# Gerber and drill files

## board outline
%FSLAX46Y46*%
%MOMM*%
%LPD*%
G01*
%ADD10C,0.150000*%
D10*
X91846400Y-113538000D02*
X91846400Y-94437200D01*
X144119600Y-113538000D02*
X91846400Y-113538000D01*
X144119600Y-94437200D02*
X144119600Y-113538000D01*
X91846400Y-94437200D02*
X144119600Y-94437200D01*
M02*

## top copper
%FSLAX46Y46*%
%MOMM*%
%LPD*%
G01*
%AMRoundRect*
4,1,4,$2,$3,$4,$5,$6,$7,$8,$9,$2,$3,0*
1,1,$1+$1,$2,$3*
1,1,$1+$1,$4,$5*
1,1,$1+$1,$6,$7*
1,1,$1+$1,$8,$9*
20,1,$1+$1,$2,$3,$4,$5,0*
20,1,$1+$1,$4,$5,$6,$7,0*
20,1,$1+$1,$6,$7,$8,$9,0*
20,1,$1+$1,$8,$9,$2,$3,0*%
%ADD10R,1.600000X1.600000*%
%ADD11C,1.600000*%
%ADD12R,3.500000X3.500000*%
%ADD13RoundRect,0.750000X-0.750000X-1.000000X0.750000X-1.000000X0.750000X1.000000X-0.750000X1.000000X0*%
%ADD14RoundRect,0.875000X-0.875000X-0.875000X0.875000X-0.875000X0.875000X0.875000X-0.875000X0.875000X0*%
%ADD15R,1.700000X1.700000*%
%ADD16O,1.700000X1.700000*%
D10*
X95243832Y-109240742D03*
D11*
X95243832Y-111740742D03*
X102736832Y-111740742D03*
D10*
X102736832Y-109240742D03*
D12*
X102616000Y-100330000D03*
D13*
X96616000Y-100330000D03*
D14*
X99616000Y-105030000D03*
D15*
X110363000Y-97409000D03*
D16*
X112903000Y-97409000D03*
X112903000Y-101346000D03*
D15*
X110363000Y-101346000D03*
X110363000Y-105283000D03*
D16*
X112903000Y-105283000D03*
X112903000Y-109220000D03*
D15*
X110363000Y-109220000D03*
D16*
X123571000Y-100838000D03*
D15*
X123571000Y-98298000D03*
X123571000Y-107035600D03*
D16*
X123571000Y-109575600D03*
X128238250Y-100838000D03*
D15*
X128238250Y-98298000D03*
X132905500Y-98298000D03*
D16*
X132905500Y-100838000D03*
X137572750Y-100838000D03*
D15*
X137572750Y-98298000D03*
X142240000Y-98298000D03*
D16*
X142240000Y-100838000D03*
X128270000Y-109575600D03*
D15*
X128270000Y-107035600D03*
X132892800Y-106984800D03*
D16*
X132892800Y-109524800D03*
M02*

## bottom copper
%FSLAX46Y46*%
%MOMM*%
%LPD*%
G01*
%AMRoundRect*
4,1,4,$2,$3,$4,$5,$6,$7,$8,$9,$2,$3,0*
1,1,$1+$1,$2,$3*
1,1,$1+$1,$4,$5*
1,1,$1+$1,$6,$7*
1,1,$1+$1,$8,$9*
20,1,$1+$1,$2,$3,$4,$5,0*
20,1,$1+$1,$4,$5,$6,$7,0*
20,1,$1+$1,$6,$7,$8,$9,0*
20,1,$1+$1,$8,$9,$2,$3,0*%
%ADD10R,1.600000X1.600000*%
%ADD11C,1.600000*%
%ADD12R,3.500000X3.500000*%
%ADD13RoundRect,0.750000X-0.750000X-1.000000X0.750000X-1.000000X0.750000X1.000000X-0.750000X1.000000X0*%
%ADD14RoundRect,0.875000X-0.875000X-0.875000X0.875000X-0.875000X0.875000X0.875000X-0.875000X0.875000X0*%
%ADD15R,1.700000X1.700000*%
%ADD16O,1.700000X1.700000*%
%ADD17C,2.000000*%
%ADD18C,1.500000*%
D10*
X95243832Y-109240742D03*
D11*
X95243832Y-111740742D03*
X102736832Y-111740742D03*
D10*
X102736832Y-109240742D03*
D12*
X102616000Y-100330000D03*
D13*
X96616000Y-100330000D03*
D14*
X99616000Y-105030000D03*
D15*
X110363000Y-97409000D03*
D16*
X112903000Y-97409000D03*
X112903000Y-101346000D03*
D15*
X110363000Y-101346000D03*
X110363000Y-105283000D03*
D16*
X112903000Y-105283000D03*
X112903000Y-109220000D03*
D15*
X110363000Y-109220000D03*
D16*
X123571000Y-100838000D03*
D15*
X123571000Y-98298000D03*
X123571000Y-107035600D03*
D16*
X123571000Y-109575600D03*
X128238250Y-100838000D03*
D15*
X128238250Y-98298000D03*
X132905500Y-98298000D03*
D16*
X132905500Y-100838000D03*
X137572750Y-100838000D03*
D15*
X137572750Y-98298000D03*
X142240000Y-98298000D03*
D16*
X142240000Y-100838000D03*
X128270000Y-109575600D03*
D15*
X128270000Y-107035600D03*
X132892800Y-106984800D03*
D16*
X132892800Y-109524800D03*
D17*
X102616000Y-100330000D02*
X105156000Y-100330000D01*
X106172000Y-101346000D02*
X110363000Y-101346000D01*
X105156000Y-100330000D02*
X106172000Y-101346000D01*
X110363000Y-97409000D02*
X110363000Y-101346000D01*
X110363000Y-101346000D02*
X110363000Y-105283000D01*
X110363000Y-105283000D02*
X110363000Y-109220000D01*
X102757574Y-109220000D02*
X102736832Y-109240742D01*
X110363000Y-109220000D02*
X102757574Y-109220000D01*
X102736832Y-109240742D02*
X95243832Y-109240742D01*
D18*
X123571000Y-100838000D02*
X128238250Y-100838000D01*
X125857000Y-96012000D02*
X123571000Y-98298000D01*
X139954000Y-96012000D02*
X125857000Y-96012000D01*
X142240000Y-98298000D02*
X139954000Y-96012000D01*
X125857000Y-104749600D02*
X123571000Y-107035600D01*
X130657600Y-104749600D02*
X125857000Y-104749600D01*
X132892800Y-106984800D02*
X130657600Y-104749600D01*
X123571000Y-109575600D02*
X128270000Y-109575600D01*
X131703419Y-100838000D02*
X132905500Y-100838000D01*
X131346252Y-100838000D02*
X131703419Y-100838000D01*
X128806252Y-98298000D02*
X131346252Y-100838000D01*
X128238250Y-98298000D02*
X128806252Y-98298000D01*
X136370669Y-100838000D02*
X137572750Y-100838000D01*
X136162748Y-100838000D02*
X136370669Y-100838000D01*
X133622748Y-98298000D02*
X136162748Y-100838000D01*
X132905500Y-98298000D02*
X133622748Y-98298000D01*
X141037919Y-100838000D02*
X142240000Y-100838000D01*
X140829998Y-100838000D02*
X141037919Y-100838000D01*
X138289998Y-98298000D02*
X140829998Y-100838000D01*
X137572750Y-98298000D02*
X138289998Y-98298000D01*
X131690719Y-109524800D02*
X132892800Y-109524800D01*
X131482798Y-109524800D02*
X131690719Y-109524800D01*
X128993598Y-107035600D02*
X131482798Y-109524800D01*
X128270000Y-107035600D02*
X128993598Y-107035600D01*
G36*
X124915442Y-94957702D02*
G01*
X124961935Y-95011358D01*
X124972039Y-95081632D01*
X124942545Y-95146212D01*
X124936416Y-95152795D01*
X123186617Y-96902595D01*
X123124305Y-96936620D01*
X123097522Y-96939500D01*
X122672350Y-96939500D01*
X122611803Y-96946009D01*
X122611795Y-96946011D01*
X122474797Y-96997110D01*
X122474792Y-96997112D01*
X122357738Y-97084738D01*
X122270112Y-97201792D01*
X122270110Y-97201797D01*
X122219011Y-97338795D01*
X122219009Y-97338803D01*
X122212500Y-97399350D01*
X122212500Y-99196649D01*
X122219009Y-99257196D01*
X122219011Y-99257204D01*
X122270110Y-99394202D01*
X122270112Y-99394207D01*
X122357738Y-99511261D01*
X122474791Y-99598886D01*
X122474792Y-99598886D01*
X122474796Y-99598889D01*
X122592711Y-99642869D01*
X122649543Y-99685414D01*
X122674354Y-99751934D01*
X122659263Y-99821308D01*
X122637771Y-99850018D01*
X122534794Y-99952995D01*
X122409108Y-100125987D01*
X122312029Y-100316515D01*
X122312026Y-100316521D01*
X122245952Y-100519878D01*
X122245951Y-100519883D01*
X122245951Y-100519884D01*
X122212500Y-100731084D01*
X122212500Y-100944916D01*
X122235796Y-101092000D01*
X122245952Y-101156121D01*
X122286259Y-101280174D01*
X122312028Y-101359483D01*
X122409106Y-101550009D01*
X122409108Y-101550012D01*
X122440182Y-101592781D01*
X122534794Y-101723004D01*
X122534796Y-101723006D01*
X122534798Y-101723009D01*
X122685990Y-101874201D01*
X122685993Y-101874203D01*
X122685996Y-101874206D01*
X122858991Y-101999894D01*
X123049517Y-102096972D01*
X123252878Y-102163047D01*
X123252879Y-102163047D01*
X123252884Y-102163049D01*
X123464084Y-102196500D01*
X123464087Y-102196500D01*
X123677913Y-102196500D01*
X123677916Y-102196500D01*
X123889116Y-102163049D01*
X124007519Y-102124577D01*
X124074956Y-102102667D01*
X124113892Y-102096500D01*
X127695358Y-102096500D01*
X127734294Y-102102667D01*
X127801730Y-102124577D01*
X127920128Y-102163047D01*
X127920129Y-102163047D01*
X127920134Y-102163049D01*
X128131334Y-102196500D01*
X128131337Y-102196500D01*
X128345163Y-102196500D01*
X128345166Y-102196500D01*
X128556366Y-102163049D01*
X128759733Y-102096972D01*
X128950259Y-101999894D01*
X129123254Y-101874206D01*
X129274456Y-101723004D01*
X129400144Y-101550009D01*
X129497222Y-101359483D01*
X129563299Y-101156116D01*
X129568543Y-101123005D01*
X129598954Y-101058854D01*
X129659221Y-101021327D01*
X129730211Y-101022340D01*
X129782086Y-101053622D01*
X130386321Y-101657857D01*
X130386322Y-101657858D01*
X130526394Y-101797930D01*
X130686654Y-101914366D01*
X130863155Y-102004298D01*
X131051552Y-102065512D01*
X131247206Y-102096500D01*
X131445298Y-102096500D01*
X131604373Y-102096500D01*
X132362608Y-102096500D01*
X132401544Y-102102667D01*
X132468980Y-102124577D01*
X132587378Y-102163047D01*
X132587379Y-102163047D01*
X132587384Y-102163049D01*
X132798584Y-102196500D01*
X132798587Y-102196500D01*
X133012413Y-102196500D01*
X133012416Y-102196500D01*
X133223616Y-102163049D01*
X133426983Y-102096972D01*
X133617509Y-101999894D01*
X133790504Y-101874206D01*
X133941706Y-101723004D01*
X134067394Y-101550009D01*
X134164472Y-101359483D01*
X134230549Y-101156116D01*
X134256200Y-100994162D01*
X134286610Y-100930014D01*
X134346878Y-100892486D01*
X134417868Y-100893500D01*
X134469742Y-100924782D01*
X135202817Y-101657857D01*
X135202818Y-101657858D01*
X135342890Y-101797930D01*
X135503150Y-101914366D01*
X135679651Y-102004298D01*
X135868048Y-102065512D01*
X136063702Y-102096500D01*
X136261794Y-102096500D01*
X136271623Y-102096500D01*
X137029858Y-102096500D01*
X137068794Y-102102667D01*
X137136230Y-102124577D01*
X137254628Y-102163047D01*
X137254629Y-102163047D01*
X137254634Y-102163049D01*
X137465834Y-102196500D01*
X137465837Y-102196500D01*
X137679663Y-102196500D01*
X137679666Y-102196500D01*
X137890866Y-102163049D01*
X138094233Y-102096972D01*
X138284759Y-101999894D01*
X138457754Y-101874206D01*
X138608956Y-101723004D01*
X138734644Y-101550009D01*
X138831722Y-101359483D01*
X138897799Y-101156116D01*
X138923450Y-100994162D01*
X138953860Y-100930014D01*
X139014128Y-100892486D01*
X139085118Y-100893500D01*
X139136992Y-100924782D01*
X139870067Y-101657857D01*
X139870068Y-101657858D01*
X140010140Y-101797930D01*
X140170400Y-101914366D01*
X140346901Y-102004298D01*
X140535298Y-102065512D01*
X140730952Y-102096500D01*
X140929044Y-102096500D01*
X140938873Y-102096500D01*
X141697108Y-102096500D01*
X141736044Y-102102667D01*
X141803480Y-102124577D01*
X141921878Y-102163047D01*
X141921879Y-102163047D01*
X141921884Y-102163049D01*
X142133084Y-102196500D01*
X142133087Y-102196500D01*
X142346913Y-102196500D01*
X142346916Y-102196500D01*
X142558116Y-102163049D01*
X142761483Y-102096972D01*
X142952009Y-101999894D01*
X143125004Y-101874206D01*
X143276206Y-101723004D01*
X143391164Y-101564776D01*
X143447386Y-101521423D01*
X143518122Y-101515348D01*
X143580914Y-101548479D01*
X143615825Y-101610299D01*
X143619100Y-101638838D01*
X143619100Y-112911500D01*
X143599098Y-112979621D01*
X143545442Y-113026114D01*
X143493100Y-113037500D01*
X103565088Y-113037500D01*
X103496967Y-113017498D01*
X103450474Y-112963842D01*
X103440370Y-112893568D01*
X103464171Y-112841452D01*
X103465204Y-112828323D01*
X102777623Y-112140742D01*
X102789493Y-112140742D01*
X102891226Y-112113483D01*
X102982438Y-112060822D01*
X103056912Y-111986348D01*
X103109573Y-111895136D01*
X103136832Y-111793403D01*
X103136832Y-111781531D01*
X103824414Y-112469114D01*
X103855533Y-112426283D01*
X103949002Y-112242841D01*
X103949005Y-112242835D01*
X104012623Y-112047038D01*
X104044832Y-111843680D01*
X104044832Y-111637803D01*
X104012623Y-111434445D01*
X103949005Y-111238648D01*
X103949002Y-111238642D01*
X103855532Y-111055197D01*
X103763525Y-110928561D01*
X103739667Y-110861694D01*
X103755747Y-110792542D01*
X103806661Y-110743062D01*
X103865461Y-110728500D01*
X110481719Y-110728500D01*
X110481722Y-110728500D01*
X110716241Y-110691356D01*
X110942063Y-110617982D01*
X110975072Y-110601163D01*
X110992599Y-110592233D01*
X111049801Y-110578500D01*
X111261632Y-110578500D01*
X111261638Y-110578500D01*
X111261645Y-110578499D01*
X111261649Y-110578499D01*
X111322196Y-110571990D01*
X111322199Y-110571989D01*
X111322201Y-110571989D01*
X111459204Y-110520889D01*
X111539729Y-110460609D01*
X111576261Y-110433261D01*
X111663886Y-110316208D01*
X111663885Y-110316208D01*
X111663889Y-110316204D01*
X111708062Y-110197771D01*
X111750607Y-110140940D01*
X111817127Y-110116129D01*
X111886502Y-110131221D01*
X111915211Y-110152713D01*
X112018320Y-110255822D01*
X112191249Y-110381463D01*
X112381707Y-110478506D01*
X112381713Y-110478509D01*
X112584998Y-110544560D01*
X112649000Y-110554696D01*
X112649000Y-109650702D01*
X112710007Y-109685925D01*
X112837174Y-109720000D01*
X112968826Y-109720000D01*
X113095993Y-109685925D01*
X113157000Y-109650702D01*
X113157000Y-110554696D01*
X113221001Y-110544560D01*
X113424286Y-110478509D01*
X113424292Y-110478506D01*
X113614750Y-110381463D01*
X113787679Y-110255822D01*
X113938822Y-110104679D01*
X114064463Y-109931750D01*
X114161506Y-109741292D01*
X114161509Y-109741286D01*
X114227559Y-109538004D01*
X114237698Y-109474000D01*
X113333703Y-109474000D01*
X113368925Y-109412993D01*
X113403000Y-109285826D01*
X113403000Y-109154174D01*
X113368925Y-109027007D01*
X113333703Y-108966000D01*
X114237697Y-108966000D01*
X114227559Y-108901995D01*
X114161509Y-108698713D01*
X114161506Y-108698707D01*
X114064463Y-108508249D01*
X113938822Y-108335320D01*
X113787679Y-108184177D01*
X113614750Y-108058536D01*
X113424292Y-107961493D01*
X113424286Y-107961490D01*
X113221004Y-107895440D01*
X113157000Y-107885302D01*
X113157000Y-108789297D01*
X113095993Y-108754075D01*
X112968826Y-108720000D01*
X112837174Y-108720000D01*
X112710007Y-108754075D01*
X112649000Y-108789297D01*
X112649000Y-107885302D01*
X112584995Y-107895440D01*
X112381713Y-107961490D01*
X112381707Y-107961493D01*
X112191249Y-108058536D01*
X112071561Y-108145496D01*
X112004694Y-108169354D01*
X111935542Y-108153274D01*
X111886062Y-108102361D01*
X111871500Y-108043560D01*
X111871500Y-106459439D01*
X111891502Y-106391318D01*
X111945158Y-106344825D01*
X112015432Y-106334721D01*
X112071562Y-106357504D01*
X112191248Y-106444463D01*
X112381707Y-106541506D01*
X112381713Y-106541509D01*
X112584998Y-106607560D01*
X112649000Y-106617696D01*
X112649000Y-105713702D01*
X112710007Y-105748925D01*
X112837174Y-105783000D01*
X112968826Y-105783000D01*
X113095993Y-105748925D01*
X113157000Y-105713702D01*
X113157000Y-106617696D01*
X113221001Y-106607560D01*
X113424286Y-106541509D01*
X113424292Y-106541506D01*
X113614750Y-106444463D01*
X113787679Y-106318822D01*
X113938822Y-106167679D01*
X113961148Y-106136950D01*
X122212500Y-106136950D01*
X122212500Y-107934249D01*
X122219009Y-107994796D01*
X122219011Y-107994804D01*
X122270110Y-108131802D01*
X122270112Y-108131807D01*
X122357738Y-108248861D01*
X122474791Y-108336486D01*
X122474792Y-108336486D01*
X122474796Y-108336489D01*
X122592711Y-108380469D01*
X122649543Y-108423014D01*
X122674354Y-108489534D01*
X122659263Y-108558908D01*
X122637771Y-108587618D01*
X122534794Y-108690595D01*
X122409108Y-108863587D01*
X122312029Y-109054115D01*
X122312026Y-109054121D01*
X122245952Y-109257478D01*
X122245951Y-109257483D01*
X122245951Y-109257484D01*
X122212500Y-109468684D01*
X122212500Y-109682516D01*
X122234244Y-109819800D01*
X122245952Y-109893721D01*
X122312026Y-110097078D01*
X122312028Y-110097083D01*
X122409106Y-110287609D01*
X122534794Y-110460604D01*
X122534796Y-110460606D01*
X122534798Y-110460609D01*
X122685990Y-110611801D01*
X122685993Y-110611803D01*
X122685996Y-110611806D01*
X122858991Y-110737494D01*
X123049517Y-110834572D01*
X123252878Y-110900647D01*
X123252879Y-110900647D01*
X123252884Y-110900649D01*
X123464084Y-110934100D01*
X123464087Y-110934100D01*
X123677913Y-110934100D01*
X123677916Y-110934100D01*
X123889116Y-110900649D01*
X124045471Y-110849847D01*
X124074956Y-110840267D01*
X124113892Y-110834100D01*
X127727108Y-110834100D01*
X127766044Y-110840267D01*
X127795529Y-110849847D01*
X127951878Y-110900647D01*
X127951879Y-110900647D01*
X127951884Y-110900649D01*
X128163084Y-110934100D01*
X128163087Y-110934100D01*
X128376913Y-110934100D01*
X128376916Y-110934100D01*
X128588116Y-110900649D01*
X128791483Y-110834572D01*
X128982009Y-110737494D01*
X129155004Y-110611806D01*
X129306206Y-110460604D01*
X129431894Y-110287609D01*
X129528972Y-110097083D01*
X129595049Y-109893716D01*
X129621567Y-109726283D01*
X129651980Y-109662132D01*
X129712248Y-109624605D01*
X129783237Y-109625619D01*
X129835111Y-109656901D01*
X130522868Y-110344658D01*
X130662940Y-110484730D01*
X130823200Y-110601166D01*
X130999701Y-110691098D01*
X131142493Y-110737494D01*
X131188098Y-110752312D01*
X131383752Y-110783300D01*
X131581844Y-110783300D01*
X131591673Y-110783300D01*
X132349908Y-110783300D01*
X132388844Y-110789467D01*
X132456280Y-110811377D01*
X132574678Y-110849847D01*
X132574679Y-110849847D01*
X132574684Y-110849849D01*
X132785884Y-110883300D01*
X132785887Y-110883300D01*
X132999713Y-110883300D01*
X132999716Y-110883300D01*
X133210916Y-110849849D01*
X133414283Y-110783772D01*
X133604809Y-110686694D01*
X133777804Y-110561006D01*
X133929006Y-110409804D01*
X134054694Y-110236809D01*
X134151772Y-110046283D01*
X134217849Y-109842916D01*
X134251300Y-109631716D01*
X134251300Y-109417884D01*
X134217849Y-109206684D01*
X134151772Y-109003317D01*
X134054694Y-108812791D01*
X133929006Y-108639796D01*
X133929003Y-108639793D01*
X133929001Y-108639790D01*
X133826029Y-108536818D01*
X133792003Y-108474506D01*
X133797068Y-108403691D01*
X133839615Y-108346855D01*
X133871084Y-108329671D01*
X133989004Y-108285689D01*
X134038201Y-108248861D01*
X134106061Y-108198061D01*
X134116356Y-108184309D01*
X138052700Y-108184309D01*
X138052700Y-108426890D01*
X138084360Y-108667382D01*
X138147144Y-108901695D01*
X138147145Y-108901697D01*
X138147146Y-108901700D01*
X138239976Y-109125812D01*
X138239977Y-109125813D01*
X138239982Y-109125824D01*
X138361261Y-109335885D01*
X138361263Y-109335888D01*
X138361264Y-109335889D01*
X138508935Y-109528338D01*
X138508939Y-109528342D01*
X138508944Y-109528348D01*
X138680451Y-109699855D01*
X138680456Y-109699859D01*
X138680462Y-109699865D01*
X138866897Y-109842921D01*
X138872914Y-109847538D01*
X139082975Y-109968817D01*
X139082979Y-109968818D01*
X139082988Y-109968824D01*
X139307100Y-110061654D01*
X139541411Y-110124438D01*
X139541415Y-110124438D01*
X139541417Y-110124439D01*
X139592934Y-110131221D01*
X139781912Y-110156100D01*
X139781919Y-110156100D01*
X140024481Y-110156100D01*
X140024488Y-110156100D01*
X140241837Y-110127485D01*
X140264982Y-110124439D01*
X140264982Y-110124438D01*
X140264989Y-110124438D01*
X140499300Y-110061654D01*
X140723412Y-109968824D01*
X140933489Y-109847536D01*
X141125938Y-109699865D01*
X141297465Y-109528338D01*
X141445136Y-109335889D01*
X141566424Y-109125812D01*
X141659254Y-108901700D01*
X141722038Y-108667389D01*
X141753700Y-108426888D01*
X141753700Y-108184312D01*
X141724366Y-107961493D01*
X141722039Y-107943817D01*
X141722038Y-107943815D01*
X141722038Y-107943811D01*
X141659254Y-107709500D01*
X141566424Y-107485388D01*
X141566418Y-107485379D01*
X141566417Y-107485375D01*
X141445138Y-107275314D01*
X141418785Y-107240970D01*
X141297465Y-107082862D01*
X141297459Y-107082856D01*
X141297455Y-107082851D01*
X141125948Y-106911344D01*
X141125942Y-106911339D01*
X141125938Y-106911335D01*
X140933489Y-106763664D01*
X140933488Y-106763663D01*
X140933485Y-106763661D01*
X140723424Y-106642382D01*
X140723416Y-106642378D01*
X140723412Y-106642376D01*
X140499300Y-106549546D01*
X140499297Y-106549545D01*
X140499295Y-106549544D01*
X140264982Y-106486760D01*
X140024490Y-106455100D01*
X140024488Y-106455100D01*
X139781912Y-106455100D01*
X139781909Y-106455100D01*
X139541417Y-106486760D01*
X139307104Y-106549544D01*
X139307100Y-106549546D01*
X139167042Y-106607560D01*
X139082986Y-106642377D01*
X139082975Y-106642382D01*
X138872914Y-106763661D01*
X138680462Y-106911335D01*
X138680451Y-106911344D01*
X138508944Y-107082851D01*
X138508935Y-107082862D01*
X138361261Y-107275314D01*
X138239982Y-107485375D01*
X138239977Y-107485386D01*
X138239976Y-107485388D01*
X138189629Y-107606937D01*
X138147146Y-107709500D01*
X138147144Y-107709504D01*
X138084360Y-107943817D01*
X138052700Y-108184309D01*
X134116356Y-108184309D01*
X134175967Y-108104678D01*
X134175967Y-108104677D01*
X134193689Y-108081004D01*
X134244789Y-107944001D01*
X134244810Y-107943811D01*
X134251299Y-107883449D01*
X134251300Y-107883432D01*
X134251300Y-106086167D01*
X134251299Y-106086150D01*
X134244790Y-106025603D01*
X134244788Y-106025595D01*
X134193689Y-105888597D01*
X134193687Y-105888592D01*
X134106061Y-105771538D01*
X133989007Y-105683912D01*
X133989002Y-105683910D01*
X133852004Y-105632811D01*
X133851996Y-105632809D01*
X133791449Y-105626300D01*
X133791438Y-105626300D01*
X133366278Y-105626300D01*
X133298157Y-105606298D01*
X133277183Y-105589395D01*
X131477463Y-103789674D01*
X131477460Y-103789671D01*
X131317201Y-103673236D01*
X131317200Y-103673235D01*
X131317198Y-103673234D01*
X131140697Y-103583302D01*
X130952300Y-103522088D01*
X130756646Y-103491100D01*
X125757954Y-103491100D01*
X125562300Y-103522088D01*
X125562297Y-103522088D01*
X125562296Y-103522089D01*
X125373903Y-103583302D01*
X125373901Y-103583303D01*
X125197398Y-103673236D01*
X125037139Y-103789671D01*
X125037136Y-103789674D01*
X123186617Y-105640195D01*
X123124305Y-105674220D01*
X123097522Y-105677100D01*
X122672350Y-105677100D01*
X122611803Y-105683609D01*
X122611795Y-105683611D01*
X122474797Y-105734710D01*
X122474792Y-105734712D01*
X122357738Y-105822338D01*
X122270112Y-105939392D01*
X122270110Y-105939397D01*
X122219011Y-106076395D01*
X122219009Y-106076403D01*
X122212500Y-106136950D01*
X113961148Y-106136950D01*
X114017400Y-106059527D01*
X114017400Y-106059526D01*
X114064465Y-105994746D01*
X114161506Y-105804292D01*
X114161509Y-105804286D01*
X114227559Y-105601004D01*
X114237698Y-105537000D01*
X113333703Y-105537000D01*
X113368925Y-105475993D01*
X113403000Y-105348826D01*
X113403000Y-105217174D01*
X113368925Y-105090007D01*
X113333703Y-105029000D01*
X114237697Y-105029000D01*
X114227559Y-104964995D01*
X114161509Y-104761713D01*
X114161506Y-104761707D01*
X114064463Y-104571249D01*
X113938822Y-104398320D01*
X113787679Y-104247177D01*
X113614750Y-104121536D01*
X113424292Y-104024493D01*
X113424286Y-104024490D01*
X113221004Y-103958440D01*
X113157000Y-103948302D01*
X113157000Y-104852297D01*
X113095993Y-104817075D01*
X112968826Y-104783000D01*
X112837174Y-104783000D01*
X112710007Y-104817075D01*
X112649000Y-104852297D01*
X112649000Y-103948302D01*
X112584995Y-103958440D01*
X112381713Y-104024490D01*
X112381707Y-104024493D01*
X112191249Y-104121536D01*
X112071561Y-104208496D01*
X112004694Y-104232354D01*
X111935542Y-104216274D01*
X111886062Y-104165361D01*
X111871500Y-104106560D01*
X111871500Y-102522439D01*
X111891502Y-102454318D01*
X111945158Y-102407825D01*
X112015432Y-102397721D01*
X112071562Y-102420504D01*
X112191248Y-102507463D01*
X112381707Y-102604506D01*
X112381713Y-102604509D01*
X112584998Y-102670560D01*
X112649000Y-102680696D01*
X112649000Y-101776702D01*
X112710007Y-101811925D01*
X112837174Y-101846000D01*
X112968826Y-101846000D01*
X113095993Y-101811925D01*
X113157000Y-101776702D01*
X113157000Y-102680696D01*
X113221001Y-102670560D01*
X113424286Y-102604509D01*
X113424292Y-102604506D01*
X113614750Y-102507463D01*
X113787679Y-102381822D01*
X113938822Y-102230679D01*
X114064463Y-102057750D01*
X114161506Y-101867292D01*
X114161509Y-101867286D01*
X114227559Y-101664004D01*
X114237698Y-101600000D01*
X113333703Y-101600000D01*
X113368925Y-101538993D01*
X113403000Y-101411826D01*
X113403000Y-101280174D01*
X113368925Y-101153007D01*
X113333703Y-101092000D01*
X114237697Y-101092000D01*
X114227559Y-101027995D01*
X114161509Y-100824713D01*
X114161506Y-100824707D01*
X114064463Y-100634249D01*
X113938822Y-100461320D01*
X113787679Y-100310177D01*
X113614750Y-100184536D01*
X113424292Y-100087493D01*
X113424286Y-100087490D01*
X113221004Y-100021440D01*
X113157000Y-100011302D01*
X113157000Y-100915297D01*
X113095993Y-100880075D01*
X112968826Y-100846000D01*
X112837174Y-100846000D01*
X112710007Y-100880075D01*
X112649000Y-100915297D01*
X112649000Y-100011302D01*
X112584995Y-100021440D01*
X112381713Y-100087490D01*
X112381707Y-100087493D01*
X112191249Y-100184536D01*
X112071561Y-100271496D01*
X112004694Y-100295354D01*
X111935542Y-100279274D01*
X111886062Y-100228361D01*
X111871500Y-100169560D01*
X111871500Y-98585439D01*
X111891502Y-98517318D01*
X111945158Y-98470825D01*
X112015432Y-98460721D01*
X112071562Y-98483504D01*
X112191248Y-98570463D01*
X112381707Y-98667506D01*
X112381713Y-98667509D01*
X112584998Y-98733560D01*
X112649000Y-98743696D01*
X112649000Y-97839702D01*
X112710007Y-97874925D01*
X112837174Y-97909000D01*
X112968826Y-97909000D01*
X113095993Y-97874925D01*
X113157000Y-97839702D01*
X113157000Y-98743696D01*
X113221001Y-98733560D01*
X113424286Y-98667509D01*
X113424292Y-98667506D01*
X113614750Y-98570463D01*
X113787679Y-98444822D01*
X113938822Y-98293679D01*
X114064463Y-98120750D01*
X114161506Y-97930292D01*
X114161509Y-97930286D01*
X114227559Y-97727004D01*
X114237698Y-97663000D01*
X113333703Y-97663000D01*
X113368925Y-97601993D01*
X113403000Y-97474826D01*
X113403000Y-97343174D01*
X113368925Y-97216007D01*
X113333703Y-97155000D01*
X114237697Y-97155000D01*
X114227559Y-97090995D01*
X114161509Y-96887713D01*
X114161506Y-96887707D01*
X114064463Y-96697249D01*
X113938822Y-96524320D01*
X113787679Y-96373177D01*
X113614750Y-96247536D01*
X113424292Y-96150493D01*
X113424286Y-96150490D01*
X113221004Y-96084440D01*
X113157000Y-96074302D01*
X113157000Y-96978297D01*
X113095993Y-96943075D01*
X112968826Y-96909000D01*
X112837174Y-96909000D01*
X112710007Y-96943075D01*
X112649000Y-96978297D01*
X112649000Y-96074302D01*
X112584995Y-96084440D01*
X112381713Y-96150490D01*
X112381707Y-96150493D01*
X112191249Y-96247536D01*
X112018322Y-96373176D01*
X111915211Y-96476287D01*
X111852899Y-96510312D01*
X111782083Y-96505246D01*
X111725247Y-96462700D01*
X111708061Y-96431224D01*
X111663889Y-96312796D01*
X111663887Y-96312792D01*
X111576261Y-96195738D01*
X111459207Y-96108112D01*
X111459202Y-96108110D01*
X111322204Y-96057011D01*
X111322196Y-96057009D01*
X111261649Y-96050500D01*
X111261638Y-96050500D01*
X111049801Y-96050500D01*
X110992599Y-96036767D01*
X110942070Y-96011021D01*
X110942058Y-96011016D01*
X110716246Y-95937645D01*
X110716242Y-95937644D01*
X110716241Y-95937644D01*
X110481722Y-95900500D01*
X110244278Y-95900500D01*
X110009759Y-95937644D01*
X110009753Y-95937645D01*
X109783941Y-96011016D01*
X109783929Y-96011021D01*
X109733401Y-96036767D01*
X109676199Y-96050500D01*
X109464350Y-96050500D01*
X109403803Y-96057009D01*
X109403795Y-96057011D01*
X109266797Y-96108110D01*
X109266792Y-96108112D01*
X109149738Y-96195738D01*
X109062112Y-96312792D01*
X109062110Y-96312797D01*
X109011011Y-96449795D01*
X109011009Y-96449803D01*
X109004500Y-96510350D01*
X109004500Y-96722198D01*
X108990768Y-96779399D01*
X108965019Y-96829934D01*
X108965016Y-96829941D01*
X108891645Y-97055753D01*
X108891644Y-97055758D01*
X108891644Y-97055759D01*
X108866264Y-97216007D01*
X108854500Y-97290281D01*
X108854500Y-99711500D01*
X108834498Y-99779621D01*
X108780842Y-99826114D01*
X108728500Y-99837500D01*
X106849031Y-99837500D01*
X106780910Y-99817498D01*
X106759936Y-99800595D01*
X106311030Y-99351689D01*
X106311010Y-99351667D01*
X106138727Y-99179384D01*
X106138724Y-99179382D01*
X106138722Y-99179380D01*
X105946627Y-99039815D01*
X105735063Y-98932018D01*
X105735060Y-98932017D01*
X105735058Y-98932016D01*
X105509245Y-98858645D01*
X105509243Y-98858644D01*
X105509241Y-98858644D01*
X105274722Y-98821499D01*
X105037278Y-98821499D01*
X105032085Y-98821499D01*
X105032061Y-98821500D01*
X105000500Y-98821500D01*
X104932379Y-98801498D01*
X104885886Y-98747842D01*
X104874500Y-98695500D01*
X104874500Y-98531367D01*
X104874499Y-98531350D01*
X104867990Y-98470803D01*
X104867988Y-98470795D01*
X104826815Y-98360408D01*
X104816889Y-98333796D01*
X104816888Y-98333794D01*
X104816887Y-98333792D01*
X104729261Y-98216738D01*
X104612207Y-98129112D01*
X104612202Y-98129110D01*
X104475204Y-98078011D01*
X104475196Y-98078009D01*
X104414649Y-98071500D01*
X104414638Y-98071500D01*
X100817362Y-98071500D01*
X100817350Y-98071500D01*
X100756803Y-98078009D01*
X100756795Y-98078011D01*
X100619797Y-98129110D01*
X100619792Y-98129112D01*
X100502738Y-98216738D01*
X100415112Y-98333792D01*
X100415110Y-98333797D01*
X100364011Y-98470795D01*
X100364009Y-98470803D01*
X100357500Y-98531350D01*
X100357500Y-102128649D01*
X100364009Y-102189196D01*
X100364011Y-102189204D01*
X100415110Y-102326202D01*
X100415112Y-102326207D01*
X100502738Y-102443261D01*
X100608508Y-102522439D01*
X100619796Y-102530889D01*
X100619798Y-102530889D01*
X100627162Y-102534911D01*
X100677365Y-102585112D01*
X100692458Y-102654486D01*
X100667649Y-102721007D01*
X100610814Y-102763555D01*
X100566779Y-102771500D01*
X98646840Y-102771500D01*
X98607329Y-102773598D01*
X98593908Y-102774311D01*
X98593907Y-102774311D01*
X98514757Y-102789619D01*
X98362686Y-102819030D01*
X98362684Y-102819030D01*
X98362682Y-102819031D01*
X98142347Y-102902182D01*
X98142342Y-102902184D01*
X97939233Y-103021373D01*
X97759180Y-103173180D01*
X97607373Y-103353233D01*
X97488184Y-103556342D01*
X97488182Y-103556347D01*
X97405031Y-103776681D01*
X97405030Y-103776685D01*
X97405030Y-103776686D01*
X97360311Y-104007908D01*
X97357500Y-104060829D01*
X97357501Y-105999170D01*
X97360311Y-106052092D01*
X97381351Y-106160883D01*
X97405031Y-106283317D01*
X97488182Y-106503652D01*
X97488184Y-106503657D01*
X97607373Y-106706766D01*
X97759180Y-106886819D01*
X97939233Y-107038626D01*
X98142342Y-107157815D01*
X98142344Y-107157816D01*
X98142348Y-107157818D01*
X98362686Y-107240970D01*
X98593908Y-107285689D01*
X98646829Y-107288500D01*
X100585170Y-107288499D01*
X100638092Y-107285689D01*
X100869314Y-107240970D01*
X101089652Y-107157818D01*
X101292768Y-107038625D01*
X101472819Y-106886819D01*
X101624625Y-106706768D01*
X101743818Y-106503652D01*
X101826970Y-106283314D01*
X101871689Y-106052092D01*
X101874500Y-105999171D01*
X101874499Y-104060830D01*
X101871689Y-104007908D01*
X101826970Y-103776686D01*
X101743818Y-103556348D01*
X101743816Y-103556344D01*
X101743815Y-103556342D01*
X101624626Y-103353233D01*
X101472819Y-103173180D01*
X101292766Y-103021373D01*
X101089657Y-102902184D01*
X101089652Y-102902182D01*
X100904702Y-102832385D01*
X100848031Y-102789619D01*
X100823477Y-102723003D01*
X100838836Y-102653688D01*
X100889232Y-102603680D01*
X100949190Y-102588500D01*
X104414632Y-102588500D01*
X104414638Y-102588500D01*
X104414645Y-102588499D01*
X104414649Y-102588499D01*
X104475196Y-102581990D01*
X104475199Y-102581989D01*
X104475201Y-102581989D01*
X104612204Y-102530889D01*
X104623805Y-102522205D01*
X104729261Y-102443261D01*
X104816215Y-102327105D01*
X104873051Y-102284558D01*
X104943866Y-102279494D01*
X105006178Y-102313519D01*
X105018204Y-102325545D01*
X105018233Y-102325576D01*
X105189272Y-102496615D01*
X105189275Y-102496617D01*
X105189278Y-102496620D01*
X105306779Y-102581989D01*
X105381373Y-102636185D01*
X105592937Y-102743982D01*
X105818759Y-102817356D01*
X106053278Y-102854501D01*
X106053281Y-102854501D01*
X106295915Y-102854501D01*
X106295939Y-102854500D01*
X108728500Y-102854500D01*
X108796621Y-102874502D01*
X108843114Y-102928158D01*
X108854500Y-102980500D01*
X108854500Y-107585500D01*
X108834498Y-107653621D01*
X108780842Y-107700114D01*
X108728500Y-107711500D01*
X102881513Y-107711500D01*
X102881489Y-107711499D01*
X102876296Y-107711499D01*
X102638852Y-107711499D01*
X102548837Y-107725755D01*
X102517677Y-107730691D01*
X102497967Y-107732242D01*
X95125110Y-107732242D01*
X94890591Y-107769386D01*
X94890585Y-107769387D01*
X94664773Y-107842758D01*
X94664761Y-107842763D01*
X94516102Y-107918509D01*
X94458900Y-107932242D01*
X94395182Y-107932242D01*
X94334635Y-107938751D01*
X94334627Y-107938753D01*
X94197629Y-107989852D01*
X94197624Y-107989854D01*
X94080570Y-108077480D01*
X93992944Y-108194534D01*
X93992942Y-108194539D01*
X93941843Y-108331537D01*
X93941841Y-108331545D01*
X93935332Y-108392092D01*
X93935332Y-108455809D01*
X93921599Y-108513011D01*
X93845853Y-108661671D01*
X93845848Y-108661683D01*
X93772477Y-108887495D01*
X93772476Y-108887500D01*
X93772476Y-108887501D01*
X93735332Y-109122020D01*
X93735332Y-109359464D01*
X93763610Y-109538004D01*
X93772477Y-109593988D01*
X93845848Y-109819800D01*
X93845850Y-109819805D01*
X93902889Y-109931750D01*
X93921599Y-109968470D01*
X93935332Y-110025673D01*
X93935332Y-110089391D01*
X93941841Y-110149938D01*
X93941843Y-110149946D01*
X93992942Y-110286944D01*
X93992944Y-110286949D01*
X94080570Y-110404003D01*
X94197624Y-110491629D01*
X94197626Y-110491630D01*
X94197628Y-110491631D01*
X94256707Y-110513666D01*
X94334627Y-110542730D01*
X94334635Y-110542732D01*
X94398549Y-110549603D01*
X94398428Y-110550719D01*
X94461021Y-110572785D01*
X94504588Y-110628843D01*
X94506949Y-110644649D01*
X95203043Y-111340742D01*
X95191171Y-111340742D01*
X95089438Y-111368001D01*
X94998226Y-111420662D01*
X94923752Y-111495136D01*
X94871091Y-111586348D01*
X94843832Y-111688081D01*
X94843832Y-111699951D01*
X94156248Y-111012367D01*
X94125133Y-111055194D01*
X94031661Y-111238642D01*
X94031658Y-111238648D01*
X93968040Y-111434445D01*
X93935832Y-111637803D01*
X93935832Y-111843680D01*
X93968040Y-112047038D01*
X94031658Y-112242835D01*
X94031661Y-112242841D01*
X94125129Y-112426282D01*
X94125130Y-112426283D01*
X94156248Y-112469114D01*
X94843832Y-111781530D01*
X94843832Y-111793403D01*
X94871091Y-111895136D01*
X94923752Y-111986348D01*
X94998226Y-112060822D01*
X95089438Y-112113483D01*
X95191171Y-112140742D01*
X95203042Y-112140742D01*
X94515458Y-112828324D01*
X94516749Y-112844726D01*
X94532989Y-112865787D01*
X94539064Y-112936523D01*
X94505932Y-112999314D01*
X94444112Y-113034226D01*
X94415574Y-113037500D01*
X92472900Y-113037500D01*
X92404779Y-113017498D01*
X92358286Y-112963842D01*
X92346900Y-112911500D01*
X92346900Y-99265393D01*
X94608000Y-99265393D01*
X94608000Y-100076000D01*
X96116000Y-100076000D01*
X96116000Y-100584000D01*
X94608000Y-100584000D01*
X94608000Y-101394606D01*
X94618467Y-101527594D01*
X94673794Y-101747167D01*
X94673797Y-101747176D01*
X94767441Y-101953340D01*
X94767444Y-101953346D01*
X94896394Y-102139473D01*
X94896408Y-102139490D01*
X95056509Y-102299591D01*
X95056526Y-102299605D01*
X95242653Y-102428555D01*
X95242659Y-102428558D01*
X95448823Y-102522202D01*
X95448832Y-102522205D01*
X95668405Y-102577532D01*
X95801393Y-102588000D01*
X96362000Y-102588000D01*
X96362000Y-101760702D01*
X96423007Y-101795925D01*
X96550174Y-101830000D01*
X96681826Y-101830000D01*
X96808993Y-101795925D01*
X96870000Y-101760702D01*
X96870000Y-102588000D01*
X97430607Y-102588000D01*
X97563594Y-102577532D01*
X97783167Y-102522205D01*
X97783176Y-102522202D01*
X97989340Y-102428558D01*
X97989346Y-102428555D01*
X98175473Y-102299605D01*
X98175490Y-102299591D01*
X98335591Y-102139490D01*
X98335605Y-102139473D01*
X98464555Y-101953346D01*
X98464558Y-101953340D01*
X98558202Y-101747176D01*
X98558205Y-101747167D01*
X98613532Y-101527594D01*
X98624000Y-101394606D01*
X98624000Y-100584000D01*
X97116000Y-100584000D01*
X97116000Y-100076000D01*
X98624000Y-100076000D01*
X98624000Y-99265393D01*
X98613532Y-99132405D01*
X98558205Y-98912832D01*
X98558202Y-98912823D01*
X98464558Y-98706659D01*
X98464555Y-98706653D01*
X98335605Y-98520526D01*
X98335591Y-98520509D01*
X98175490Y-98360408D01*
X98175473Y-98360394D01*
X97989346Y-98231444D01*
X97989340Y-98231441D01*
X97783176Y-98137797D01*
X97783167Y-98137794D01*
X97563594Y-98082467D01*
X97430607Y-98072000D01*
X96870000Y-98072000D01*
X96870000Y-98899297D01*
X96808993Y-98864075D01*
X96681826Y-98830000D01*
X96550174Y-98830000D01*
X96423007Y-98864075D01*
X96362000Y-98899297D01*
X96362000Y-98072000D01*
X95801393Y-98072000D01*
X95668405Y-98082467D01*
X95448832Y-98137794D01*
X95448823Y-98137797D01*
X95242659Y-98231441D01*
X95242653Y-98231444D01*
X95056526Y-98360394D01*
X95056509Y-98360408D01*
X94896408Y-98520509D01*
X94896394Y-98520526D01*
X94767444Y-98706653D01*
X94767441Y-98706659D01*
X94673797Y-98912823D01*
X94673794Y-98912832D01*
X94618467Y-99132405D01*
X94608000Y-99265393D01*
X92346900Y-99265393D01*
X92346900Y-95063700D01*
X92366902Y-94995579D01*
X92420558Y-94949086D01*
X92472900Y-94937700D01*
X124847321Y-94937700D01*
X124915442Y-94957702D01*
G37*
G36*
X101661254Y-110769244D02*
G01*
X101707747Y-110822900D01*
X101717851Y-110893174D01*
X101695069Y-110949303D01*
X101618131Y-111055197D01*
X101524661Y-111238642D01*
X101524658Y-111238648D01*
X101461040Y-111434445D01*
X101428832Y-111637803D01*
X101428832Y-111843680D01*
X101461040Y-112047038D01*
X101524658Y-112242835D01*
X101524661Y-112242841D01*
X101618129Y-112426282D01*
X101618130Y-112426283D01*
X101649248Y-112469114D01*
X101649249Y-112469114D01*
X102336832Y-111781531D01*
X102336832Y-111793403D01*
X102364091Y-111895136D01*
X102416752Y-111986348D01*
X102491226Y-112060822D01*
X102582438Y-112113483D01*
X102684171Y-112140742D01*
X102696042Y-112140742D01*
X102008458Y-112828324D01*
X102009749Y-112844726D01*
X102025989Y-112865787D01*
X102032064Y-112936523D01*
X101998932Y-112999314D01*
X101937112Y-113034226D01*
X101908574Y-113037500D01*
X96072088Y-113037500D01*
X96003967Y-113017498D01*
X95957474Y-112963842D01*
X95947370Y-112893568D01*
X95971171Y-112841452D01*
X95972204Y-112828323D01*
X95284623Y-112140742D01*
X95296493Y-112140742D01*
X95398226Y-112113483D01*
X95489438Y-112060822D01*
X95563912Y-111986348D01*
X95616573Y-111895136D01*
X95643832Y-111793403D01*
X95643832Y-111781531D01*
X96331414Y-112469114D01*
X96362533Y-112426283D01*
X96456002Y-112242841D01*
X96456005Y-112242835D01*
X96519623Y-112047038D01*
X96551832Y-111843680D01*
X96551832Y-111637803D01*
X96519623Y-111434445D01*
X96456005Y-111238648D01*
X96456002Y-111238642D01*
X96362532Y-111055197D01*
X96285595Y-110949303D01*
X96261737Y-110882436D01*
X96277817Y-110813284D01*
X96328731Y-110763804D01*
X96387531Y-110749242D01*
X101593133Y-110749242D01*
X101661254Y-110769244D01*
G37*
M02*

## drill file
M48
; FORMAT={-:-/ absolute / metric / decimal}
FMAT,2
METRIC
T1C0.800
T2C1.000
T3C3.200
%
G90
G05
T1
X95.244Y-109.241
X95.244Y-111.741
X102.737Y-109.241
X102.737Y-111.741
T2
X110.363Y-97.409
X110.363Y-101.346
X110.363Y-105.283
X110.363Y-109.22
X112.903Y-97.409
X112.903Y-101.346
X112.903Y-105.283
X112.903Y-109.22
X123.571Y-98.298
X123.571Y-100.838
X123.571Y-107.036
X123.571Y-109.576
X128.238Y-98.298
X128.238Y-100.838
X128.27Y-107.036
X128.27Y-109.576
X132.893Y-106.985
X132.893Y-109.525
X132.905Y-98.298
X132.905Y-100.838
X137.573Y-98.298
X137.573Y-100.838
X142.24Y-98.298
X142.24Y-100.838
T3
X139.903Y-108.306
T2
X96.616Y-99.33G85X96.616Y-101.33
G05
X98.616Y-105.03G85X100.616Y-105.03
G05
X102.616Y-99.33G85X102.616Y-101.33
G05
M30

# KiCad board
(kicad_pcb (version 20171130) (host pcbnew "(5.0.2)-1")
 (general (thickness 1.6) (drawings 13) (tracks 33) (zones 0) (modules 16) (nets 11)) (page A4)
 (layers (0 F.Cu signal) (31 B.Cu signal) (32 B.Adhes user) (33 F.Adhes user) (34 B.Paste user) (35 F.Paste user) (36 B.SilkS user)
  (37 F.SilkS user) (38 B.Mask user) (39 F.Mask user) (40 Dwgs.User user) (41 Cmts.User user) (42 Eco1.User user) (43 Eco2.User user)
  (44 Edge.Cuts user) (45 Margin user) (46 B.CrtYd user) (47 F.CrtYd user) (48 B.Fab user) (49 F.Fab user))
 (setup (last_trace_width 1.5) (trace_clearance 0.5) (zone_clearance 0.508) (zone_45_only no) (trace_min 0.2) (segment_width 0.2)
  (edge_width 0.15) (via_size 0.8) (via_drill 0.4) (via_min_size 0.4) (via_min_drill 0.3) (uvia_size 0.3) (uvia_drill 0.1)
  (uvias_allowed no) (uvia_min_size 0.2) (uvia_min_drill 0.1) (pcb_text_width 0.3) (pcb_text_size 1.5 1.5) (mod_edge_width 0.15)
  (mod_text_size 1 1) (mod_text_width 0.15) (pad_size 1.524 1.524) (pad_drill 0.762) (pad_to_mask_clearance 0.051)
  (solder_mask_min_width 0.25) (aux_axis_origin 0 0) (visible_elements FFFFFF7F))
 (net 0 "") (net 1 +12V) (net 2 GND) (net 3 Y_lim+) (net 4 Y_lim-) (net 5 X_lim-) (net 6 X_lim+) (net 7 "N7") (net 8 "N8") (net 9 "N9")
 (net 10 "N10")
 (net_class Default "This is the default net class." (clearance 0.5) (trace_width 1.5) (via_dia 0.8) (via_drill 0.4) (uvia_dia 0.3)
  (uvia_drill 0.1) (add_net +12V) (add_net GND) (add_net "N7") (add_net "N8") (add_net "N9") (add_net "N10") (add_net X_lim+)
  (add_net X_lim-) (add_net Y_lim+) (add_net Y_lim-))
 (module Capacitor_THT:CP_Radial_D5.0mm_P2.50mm (layer F.Cu) (at 95.243832 109.240742 270)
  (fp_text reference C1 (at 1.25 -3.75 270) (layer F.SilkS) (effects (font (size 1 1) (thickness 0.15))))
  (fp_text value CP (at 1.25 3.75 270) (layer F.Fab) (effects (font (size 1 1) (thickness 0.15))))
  (pad 1 thru_hole rect (at 0 0 270) (size 1.6 1.6) (drill 0.8) (layers *.Cu *.Mask) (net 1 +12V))
  (pad 2 thru_hole circle (at 2.5 0 270) (size 1.6 1.6) (drill 0.8) (layers *.Cu *.Mask) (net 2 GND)))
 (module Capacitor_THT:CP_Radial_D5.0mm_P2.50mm (layer F.Cu) (at 102.736832 109.240742 270)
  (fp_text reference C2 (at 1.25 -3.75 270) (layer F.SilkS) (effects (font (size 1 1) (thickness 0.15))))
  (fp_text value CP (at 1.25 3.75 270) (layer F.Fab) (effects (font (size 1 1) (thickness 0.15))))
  (pad 2 thru_hole circle (at 2.5 0 270) (size 1.6 1.6) (drill 0.8) (layers *.Cu *.Mask) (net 2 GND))
  (pad 1 thru_hole rect (at 0 0 270) (size 1.6 1.6) (drill 0.8) (layers *.Cu *.Mask) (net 1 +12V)))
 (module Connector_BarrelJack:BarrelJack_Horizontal (layer F.Cu) (at 102.616 100.33)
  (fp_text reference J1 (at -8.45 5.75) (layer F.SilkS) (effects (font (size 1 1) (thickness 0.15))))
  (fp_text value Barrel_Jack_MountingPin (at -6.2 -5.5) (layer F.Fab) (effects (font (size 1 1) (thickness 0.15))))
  (pad 1 thru_hole rect (at 0 0) (size 3.5 3.5) (drill oval 1 3) (layers *.Cu *.Mask) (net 1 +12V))
  (pad 2 thru_hole roundrect (at -6 0) (size 3 3.5) (drill oval 1 3) (layers *.Cu *.Mask) (roundrect_rratio 0.25) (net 2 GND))
  (pad 3 thru_hole roundrect (at -3 4.7) (size 3.5 3.5) (drill oval 3 1) (layers *.Cu *.Mask) (roundrect_rratio 0.25)))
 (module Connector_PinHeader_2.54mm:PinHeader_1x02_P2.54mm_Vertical (layer F.Cu) (at 110.363 97.409 90)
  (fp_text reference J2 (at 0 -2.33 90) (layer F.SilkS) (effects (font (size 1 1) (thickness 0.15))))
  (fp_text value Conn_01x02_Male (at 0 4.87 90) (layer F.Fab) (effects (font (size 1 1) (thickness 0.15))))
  (pad 1 thru_hole rect (at 0 0 90) (size 1.7 1.7) (drill 1) (layers *.Cu *.Mask) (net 1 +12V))
  (pad 2 thru_hole oval (at 0 2.54 90) (size 1.7 1.7) (drill 1) (layers *.Cu *.Mask) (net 2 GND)))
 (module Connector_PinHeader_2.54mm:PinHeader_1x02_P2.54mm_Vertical (layer F.Cu) (at 110.363 101.346 90)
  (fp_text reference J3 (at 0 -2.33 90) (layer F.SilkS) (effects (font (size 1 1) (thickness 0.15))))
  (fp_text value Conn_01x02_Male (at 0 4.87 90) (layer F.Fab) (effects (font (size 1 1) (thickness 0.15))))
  (pad 2 thru_hole oval (at 0 2.54 90) (size 1.7 1.7) (drill 1) (layers *.Cu *.Mask) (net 2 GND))
  (pad 1 thru_hole rect (at 0 0 90) (size 1.7 1.7) (drill 1) (layers *.Cu *.Mask) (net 1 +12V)))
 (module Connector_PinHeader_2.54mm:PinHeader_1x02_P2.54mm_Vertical (layer F.Cu) (at 110.363 105.283 90)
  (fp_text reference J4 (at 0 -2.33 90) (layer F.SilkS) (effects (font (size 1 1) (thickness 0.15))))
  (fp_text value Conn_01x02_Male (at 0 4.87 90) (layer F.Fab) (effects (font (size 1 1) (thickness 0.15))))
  (pad 1 thru_hole rect (at 0 0 90) (size 1.7 1.7) (drill 1) (layers *.Cu *.Mask) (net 1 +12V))
  (pad 2 thru_hole oval (at 0 2.54 90) (size 1.7 1.7) (drill 1) (layers *.Cu *.Mask) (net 2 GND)))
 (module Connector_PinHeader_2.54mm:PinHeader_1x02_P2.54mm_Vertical (layer F.Cu) (at 110.363 109.22 90)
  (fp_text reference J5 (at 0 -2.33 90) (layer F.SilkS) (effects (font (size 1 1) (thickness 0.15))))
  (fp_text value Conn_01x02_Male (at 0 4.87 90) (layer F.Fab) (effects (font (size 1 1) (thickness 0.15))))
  (pad 2 thru_hole oval (at 0 2.54 90) (size 1.7 1.7) (drill 1) (layers *.Cu *.Mask) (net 2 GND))
  (pad 1 thru_hole rect (at 0 0 90) (size 1.7 1.7) (drill 1) (layers *.Cu *.Mask) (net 1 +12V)))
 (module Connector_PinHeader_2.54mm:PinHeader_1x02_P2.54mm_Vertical (layer F.Cu) (at 123.571 98.298)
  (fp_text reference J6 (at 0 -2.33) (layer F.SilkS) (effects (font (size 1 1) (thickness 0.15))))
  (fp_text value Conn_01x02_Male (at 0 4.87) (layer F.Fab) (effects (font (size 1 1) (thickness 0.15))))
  (pad 2 thru_hole oval (at 0 2.54) (size 1.7 1.7) (drill 1) (layers *.Cu *.Mask) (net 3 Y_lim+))
  (pad 1 thru_hole rect (at 0 0) (size 1.7 1.7) (drill 1) (layers *.Cu *.Mask) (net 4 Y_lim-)))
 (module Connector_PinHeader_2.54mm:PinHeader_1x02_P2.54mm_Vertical (layer F.Cu) (at 123.571 107.0356)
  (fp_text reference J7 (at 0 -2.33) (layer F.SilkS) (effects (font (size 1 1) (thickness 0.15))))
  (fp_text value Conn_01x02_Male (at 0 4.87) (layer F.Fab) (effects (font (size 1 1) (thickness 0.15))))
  (pad 1 thru_hole rect (at 0 0) (size 1.7 1.7) (drill 1) (layers *.Cu *.Mask) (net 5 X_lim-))
  (pad 2 thru_hole oval (at 0 2.54) (size 1.7 1.7) (drill 1) (layers *.Cu *.Mask) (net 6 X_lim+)))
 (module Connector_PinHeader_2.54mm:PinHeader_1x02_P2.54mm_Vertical (layer F.Cu) (at 128.23825 98.298)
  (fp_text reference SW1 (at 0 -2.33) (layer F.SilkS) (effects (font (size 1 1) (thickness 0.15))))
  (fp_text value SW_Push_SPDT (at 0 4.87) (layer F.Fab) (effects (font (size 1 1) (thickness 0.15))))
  (pad 2 thru_hole oval (at 0 2.54) (size 1.7 1.7) (drill 1) (layers *.Cu *.Mask) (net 3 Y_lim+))
  (pad 1 thru_hole rect (at 0 0) (size 1.7 1.7) (drill 1) (layers *.Cu *.Mask) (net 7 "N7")))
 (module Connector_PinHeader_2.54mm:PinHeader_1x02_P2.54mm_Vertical (layer F.Cu) (at 132.9055 98.298)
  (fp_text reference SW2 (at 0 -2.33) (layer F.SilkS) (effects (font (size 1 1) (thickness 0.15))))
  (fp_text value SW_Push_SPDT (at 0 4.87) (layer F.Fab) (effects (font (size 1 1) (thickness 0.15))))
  (pad 1 thru_hole rect (at 0 0) (size 1.7 1.7) (drill 1) (layers *.Cu *.Mask) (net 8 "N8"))
  (pad 2 thru_hole oval (at 0 2.54) (size 1.7 1.7) (drill 1) (layers *.Cu *.Mask) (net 7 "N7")))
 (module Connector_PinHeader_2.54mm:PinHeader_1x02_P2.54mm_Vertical (layer F.Cu) (at 137.57275 98.298)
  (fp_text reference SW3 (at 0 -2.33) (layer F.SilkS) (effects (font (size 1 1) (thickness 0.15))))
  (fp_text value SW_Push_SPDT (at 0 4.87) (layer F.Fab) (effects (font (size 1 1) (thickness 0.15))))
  (pad 2 thru_hole oval (at 0 2.54) (size 1.7 1.7) (drill 1) (layers *.Cu *.Mask) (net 8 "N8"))
  (pad 1 thru_hole rect (at 0 0) (size 1.7 1.7) (drill 1) (layers *.Cu *.Mask) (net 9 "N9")))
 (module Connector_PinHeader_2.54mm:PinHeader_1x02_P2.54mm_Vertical (layer F.Cu) (at 142.24 98.298)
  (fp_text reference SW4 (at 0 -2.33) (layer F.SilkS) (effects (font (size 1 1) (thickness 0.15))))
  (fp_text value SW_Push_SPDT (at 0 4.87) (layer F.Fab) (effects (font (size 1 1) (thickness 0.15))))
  (pad 1 thru_hole rect (at 0 0) (size 1.7 1.7) (drill 1) (layers *.Cu *.Mask) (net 4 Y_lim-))
  (pad 2 thru_hole oval (at 0 2.54) (size 1.7 1.7) (drill 1) (layers *.Cu *.Mask) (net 9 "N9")))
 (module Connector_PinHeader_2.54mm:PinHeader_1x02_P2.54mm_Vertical (layer F.Cu) (at 128.27 107.0356)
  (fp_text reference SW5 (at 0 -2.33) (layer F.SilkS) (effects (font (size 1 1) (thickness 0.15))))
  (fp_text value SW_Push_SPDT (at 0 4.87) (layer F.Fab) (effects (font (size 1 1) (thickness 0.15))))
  (pad 2 thru_hole oval (at 0 2.54) (size 1.7 1.7) (drill 1) (layers *.Cu *.Mask) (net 6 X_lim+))
  (pad 1 thru_hole rect (at 0 0) (size 1.7 1.7) (drill 1) (layers *.Cu *.Mask) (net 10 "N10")))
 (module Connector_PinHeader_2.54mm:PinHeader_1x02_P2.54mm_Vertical (layer F.Cu) (at 132.8928 106.9848)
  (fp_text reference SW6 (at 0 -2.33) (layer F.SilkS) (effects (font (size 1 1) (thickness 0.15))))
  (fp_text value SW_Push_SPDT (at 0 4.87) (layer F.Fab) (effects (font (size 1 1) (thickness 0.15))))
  (pad 1 thru_hole rect (at 0 0) (size 1.7 1.7) (drill 1) (layers *.Cu *.Mask) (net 5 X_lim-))
  (pad 2 thru_hole oval (at 0 2.54) (size 1.7 1.7) (drill 1) (layers *.Cu *.Mask) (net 10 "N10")))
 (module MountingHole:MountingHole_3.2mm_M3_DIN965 (layer F.Cu) (at 139.9032 108.3056)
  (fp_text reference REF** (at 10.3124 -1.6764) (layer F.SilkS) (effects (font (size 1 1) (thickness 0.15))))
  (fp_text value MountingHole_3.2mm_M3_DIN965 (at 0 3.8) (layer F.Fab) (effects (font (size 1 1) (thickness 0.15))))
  (pad 1 np_thru_hole circle (at 0 0) (size 3.2 3.2) (drill 3.2) (layers *.Cu *.Mask)))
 (gr_line (start 91.8464 113.538) (end 91.8464 94.4372) (layer Edge.Cuts) (width 0.15))
 (gr_line (start 144.1196 113.538) (end 91.8464 113.538) (layer Edge.Cuts) (width 0.15))
 (gr_line (start 144.1196 94.4372) (end 144.1196 113.538) (layer Edge.Cuts) (width 0.15))
 (gr_line (start 91.8464 94.4372) (end 144.1196 94.4372) (layer Edge.Cuts) (width 0.15))
 (segment (start 102.616 100.33) (end 105.156 100.33) (width 2) (layer B.Cu) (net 1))
 (segment (start 106.172 101.346) (end 110.363 101.346) (width 2) (layer B.Cu) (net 1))
 (segment (start 105.156 100.33) (end 106.172 101.346) (width 2) (layer B.Cu) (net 1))
 (segment (start 110.363 97.409) (end 110.363 101.346) (width 2) (layer B.Cu) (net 1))
 (segment (start 110.363 101.346) (end 110.363 105.283) (width 2) (layer B.Cu) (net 1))
 (segment (start 110.363 105.283) (end 110.363 109.22) (width 2) (layer B.Cu) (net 1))
 (segment (start 102.757574 109.22) (end 102.736832 109.240742) (width 2) (layer B.Cu) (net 1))
 (segment (start 110.363 109.22) (end 102.757574 109.22) (width 2) (layer B.Cu) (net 1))
 (segment (start 102.736832 109.240742) (end 95.243832 109.240742) (width 2) (layer B.Cu) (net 1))
 (segment (start 123.571 100.838) (end 128.23825 100.838) (width 1.5) (layer B.Cu) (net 3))
 (segment (start 125.857 96.012) (end 123.571 98.298) (width 1.5) (layer B.Cu) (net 4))
 (segment (start 139.954 96.012) (end 125.857 96.012) (width 1.5) (layer B.Cu) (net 4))
 (segment (start 142.24 98.298) (end 139.954 96.012) (width 1.5) (layer B.Cu) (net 4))
 (segment (start 125.857 104.7496) (end 123.571 107.0356) (width 1.5) (layer B.Cu) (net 5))
 (segment (start 130.6576 104.7496) (end 125.857 104.7496) (width 1.5) (layer B.Cu) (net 5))
 (segment (start 132.8928 106.9848) (end 130.6576 104.7496) (width 1.5) (layer B.Cu) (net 5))
 (segment (start 123.571 109.5756) (end 128.27 109.5756) (width 1.5) (layer B.Cu) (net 6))
 (segment (start 131.703419 100.838) (end 132.9055 100.838) (width 1.5) (layer B.Cu) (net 7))
 (segment (start 131.346252 100.838) (end 131.703419 100.838) (width 1.5) (layer B.Cu) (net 7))
 (segment (start 128.806252 98.298) (end 131.346252 100.838) (width 1.5) (layer B.Cu) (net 7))
 (segment (start 128.23825 98.298) (end 128.806252 98.298) (width 1.5) (layer B.Cu) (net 7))
 (segment (start 136.370669 100.838) (end 137.57275 100.838) (width 1.5) (layer B.Cu) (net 8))
 (segment (start 136.162748 100.838) (end 136.370669 100.838) (width 1.5) (layer B.Cu) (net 8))
 (segment (start 133.622748 98.298) (end 136.162748 100.838) (width 1.5) (layer B.Cu) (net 8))
 (segment (start 132.9055 98.298) (end 133.622748 98.298) (width 1.5) (layer B.Cu) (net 8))
 (segment (start 141.037919 100.838) (end 142.24 100.838) (width 1.5) (layer B.Cu) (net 9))
 (segment (start 140.829998 100.838) (end 141.037919 100.838) (width 1.5) (layer B.Cu) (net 9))
 (segment (start 138.289998 98.298) (end 140.829998 100.838) (width 1.5) (layer B.Cu) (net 9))
 (segment (start 137.57275 98.298) (end 138.289998 98.298) (width 1.5) (layer B.Cu) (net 9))
 (segment (start 131.690719 109.5248) (end 132.8928 109.5248) (width 1.5) (layer B.Cu) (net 10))
 (segment (start 131.482798 109.5248) (end 131.690719 109.5248) (width 1.5) (layer B.Cu) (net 10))
 (segment (start 128.993598 107.0356) (end 131.482798 109.5248) (width 1.5) (layer B.Cu) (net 10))
 (segment (start 128.27 107.0356) (end 128.993598 107.0356) (width 1.5) (layer B.Cu) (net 10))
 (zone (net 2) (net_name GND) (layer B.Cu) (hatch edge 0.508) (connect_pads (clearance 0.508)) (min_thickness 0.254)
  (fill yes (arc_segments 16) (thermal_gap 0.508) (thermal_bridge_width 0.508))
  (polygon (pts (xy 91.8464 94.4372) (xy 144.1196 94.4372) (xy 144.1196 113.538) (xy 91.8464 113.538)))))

